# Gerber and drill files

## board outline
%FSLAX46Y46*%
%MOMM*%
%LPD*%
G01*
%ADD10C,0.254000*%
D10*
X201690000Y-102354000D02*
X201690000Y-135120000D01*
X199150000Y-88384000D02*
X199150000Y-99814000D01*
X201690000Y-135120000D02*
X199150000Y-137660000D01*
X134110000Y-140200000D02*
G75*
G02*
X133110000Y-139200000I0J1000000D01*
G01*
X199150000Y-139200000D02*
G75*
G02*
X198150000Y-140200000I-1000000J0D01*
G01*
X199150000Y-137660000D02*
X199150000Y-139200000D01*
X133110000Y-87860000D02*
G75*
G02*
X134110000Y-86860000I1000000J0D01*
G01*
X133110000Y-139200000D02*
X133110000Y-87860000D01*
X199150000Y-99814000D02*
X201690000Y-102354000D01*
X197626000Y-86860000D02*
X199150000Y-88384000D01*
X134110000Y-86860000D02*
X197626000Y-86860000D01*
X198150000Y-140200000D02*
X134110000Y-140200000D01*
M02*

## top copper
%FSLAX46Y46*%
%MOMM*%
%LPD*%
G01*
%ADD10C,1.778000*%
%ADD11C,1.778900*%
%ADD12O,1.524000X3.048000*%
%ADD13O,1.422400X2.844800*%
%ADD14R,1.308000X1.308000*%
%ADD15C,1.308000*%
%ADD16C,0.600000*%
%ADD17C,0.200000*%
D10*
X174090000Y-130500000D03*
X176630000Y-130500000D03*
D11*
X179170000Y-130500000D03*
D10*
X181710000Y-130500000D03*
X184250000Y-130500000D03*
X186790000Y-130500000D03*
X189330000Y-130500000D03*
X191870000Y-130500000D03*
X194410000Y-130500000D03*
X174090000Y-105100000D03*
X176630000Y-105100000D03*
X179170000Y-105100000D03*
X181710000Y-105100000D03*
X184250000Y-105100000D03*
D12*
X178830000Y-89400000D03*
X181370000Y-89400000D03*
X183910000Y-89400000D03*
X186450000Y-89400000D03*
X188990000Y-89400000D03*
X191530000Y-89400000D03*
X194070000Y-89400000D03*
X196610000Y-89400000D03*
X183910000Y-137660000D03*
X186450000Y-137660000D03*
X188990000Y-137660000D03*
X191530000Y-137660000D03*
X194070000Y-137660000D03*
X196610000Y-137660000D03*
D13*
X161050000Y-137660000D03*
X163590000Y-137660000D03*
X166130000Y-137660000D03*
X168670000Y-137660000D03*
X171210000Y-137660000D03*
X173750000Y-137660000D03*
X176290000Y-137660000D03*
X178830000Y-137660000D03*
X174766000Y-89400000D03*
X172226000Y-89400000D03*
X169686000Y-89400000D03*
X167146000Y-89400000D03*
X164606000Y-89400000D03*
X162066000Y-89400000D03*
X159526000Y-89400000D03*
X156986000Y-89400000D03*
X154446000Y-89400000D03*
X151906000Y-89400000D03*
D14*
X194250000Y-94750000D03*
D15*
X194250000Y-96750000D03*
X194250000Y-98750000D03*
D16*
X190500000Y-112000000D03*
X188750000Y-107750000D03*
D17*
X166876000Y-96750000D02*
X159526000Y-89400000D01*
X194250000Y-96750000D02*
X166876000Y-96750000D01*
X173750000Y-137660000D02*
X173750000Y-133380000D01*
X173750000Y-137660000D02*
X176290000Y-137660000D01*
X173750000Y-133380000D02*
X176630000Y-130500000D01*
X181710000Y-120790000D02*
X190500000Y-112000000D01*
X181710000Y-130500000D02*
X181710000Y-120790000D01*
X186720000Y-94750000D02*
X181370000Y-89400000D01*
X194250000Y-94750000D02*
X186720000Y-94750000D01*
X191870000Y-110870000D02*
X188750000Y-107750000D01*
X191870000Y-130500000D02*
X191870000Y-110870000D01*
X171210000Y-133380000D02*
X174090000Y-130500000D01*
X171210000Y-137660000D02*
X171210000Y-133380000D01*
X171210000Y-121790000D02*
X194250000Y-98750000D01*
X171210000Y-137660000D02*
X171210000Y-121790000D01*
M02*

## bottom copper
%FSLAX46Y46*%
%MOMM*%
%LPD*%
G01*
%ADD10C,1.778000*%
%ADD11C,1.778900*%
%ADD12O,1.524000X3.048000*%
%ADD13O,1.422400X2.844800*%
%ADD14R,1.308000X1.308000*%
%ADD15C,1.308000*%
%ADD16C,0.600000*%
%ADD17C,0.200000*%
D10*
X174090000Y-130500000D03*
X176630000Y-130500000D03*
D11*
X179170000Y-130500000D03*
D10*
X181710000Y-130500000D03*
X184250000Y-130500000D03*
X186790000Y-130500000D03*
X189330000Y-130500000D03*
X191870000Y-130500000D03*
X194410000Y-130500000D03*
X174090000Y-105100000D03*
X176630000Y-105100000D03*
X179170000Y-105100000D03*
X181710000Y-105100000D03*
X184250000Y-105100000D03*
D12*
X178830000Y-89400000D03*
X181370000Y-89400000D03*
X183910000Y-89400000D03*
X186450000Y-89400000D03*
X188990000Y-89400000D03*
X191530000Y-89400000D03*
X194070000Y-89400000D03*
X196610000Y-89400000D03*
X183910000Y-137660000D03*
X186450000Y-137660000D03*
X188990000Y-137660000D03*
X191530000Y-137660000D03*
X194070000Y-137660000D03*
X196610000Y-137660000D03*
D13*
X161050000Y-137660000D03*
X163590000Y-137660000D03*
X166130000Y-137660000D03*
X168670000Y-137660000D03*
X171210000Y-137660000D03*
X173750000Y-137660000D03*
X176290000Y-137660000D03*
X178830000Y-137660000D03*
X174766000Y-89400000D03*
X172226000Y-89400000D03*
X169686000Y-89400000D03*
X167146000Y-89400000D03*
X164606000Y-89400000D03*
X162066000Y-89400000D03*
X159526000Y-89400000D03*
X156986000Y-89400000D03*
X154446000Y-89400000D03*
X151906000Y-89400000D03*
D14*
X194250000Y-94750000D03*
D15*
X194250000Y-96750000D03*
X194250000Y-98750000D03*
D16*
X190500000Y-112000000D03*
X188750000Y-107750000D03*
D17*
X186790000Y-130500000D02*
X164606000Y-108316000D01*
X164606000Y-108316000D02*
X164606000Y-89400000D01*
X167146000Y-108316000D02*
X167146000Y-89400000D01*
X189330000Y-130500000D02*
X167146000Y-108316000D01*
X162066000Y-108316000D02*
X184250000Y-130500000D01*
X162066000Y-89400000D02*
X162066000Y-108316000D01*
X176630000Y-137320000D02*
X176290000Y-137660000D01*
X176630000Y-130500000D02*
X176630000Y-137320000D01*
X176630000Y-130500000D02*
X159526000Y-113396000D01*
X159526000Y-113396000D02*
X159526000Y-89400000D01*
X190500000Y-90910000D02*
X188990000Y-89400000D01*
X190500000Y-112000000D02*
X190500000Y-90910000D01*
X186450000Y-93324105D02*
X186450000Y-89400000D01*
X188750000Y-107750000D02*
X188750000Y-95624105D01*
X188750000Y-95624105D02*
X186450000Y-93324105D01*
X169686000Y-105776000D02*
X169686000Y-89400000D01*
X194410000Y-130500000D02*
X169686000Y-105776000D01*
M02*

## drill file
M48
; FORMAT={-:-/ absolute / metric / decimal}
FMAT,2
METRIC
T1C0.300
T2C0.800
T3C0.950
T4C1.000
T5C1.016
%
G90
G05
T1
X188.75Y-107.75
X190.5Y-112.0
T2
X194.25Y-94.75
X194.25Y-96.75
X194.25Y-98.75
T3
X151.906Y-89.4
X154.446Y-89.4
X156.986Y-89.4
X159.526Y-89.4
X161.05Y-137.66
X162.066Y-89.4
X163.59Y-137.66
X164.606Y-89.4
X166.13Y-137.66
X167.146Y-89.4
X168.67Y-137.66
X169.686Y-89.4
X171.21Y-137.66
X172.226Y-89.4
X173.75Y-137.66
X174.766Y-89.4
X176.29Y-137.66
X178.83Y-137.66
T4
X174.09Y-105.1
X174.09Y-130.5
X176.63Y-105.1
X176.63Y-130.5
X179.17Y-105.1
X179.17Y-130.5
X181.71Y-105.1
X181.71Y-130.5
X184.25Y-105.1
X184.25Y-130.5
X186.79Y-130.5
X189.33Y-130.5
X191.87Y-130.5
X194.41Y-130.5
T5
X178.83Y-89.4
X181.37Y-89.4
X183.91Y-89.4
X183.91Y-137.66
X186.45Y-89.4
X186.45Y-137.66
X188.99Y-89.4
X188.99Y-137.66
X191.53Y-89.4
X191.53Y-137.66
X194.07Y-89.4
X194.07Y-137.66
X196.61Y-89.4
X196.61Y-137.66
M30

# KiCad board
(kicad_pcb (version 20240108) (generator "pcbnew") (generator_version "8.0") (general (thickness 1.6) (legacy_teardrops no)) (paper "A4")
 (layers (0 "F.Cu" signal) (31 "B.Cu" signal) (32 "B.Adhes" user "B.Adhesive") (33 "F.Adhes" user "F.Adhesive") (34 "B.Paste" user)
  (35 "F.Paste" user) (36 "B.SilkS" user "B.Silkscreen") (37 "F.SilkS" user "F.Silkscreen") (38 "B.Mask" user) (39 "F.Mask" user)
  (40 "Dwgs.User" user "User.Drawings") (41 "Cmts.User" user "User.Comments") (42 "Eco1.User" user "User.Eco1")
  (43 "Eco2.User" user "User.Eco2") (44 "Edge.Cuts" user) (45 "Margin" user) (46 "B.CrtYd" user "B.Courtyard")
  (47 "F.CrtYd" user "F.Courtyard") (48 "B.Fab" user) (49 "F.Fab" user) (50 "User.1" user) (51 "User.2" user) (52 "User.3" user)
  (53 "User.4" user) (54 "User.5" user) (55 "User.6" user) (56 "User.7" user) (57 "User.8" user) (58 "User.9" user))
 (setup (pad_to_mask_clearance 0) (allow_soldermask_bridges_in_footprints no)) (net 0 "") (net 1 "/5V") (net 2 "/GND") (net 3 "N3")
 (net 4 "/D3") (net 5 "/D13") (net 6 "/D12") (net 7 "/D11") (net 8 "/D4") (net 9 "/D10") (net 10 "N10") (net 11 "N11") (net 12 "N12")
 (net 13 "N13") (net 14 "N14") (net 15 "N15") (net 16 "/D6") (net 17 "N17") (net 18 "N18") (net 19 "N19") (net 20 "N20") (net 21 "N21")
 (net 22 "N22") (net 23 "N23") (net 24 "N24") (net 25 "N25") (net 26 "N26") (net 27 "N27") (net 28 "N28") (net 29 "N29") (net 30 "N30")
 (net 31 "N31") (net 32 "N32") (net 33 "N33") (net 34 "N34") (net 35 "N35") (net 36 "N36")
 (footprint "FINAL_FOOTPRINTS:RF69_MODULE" (layer "F.Cu") (at 36.0029 13.4314)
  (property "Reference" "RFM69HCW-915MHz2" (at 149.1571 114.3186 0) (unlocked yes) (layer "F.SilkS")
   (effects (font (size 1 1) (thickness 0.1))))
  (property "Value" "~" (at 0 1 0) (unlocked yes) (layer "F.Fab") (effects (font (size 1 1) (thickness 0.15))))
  (pad "1" thru_hole circle (at 138.0871 117.0686 90) (size 1.778 1.778) (drill 1) (layers "*.Cu" "*.Mask") (remove_unused_layers no)
   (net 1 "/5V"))
  (pad "2" thru_hole circle (at 140.6271 117.0686 90) (size 1.778 1.778) (drill 1) (layers "*.Cu" "*.Mask") (remove_unused_layers no)
   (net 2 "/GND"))
  (pad "3" thru_hole circle (at 143.1671 117.0686) (size 1.7789 1.7789) (drill 1) (layers "*.Cu" "*.Mask") (remove_unused_layers no)
   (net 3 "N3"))
  (pad "4" thru_hole circle (at 145.7071 117.0686) (size 1.778 1.778) (drill 1) (layers "*.Cu" "*.Mask") (remove_unused_layers no)
   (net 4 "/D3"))
  (pad "5" thru_hole circle (at 148.2471 117.0686 90) (size 1.778 1.778) (drill 1) (layers "*.Cu" "*.Mask") (remove_unused_layers no)
   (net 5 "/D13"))
  (pad "6" thru_hole circle (at 150.7871 117.0686 90) (size 1.778 1.778) (drill 1) (layers "*.Cu" "*.Mask") (remove_unused_layers no)
   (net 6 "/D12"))
  (pad "7" thru_hole circle (at 153.3271 117.0686) (size 1.778 1.778) (drill 1) (layers "*.Cu" "*.Mask") (remove_unused_layers no)
   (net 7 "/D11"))
  (pad "8" thru_hole circle (at 155.8671 117.0686 90) (size 1.778 1.778) (drill 1) (layers "*.Cu" "*.Mask") (remove_unused_layers no)
   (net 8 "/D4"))
  (pad "9" thru_hole circle (at 158.4071 117.0686 90) (size 1.778 1.778) (drill 1) (layers "*.Cu" "*.Mask") (remove_unused_layers no)
   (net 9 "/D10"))
  (pad "10" thru_hole circle (at 138.0871 91.6686 90) (size 1.778 1.778) (drill 1) (layers "*.Cu" "*.Mask") (remove_unused_layers no)
   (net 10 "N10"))
  (pad "11" thru_hole circle (at 140.6271 91.6686 90) (size 1.778 1.778) (drill 1) (layers "*.Cu" "*.Mask") (remove_unused_layers no)
   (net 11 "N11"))
  (pad "12" thru_hole circle (at 143.1671 91.6686 90) (size 1.778 1.778) (drill 1) (layers "*.Cu" "*.Mask") (remove_unused_layers no)
   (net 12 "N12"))
  (pad "13" thru_hole circle (at 145.7071 91.6686 90) (size 1.778 1.778) (drill 1) (layers "*.Cu" "*.Mask") (remove_unused_layers no)
   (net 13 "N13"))
  (pad "14" thru_hole circle (at 148.2471 91.6686 90) (size 1.778 1.778) (drill 1) (layers "*.Cu" "*.Mask") (remove_unused_layers no)
   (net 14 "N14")))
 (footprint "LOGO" (layer "F.Cu") (at 145.75 127.75)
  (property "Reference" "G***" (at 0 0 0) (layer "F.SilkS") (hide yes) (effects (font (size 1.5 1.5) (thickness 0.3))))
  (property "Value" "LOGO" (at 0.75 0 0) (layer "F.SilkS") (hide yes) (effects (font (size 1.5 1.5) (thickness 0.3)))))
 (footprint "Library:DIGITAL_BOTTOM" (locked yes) (layer "F.Cu") (at 187.72 89.4)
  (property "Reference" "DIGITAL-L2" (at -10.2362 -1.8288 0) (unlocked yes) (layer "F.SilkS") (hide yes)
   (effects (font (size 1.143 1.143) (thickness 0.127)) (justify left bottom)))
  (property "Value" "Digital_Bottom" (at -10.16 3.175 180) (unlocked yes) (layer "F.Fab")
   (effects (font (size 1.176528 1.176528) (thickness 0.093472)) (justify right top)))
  (pad "1" thru_hole oval (at -8.89 0 90) (size 3.048 1.524) (drill 1.016) (layers "*.Cu" "*.Mask") (remove_unused_layers no) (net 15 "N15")
   (solder_mask_margin 0.0508) (thermal_bridge_angle 0))
  (pad "2" thru_hole oval (at -6.35 0 90) (size 3.048 1.524) (drill 1.016) (layers "*.Cu" "*.Mask") (remove_unused_layers no) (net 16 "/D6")
   (solder_mask_margin 0.0508) (thermal_bridge_angle 0))
  (pad "3" thru_hole oval (at -3.81 0 90) (size 3.048 1.524) (drill 1.016) (layers "*.Cu" "*.Mask") (remove_unused_layers no) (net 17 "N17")
   (solder_mask_margin 0.0508) (thermal_bridge_angle 0))
  (pad "4" thru_hole oval (at -1.27 0 90) (size 3.048 1.524) (drill 1.016) (layers "*.Cu" "*.Mask") (remove_unused_layers no) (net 8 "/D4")
   (solder_mask_margin 0.0508) (thermal_bridge_angle 0))
  (pad "5" thru_hole oval (at 1.27 0 90) (size 3.048 1.524) (drill 1.016) (layers "*.Cu" "*.Mask") (remove_unused_layers no) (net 4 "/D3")
   (solder_mask_margin 0.0508) (thermal_bridge_angle 0))
  (pad "6" thru_hole oval (at 3.81 0 90) (size 3.048 1.524) (drill 1.016) (layers "*.Cu" "*.Mask") (remove_unused_layers no) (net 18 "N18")
   (solder_mask_margin 0.0508) (thermal_bridge_angle 0))
  (pad "7" thru_hole oval (at 6.35 0 90) (size 3.048 1.524) (drill 1.016) (layers "*.Cu" "*.Mask") (remove_unused_layers no) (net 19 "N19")
   (solder_mask_margin 0.0508) (thermal_bridge_angle 0))
  (pad "8" thru_hole oval (at 8.89 0 90) (size 3.048 1.524) (drill 1.016) (layers "*.Cu" "*.Mask") (remove_unused_layers no) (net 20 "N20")
   (solder_mask_margin 0.0508) (thermal_bridge_angle 0)))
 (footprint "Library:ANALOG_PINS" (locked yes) (layer "F.Cu") (at 190.26 137.66)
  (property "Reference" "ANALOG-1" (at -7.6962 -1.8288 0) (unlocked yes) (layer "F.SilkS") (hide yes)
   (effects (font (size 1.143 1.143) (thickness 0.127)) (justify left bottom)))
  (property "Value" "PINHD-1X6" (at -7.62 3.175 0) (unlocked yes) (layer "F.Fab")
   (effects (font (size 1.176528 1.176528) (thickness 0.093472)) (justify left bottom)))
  (pad "1" thru_hole oval (at -6.35 0 90) (size 3.048 1.524) (drill 1.016) (layers "*.Cu" "*.Mask") (remove_unused_layers no) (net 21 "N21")
   (solder_mask_margin 0.0508) (thermal_bridge_angle 0))
  (pad "2" thru_hole oval (at -3.81 0 90) (size 3.048 1.524) (drill 1.016) (layers "*.Cu" "*.Mask") (remove_unused_layers no) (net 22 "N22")
   (solder_mask_margin 0.0508) (thermal_bridge_angle 0))
  (pad "3" thru_hole oval (at -1.27 0 90) (size 3.048 1.524) (drill 1.016) (layers "*.Cu" "*.Mask") (remove_unused_layers no) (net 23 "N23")
   (solder_mask_margin 0.0508) (thermal_bridge_angle 0))
  (pad "4" thru_hole oval (at 1.27 0 90) (size 3.048 1.524) (drill 1.016) (layers "*.Cu" "*.Mask") (remove_unused_layers no) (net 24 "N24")
   (solder_mask_margin 0.0508) (thermal_bridge_angle 0))
  (pad "5" thru_hole oval (at 3.81 0 90) (size 3.048 1.524) (drill 1.016) (layers "*.Cu" "*.Mask") (remove_unused_layers no) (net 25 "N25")
   (solder_mask_margin 0.0508) (thermal_bridge_angle 0))
  (pad "6" thru_hole oval (at 6.35 0 90) (size 3.048 1.524) (drill 1.016) (layers "*.Cu" "*.Mask") (remove_unused_layers no) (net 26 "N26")
   (solder_mask_margin 0.0508) (thermal_bridge_angle 0)))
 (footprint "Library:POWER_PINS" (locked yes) (layer "F.Cu") (at 169.94 137.66)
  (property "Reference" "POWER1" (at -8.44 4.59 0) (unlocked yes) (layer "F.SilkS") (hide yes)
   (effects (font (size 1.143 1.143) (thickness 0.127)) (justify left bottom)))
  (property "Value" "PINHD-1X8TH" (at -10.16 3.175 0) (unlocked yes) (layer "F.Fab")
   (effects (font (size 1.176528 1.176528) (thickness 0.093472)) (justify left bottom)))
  (pad "1" thru_hole oval (at -8.89 0 90) (size 2.8448 1.4224) (drill 0.95) (layers "*.Cu" "*.Mask") (remove_unused_layers no)
   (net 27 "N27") (solder_mask_margin 0.0508) (thermal_bridge_angle 0))
  (pad "2" thru_hole oval (at -6.35 0 90) (size 2.8448 1.4224) (drill 0.95) (layers "*.Cu" "*.Mask") (remove_unused_layers no)
   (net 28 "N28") (solder_mask_margin 0.0508) (thermal_bridge_angle 0))
  (pad "3" thru_hole oval (at -3.81 0 90) (size 2.8448 1.4224) (drill 0.95) (layers "*.Cu" "*.Mask") (remove_unused_layers no)
   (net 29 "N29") (solder_mask_margin 0.0508) (thermal_bridge_angle 0))
  (pad "4" thru_hole oval (at -1.27 0 90) (size 2.8448 1.4224) (drill 0.95) (layers "*.Cu" "*.Mask") (remove_unused_layers no)
   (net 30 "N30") (solder_mask_margin 0.0508) (thermal_bridge_angle 0))
  (pad "5" thru_hole oval (at 1.27 0 90) (size 2.8448 1.4224) (drill 0.95) (layers "*.Cu" "*.Mask") (remove_unused_layers no) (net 1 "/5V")
   (solder_mask_margin 0.0508) (thermal_bridge_angle 0))
  (pad "6" thru_hole oval (at 3.81 0 90) (size 2.8448 1.4224) (drill 0.95) (layers "*.Cu" "*.Mask") (remove_unused_layers no) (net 2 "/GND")
   (solder_mask_margin 0.0508) (thermal_bridge_angle 0))
  (pad "7" thru_hole oval (at 6.35 0 90) (size 2.8448 1.4224) (drill 0.95) (layers "*.Cu" "*.Mask") (remove_unused_layers no) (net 2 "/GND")
   (solder_mask_margin 0.0508) (thermal_bridge_angle 0))
  (pad "8" thru_hole oval (at 8.89 0 90) (size 2.8448 1.4224) (drill 0.95) (layers "*.Cu" "*.Mask") (remove_unused_layers no) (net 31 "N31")
   (solder_mask_margin 0.0508) (thermal_bridge_angle 0)))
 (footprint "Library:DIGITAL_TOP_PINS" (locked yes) (layer "F.Cu") (at 163.336 89.4 180)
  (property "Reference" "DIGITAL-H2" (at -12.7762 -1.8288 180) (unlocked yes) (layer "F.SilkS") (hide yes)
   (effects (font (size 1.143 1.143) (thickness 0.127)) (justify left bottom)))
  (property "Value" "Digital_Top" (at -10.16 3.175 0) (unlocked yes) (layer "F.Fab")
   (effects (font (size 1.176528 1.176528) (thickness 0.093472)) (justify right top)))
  (pad "1" thru_hole oval (at -11.43 0 270) (size 2.8448 1.4224) (drill 0.95) (layers "*.Cu" "*.Mask") (remove_unused_layers no)
   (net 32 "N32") (solder_mask_margin 0.0508) (thermal_bridge_angle 0))
  (pad "2" thru_hole oval (at -8.89 0 270) (size 2.8448 1.4224) (drill 0.95) (layers "*.Cu" "*.Mask") (remove_unused_layers no)
   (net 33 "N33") (solder_mask_margin 0.0508) (thermal_bridge_angle 0))
  (pad "3" thru_hole oval (at -6.35 0 270) (size 2.8448 1.4224) (drill 0.95) (layers "*.Cu" "*.Mask") (remove_unused_layers no)
   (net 9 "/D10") (solder_mask_margin 0.0508) (thermal_bridge_angle 0))
  (pad "4" thru_hole oval (at -3.81 0 270) (size 2.8448 1.4224) (drill 0.95) (layers "*.Cu" "*.Mask") (remove_unused_layers no)
   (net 7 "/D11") (solder_mask_margin 0.0508) (thermal_bridge_angle 0))
  (pad "5" thru_hole oval (at -1.27 0 270) (size 2.8448 1.4224) (drill 0.95) (layers "*.Cu" "*.Mask") (remove_unused_layers no)
   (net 6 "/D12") (solder_mask_margin 0.0508) (thermal_bridge_angle 0))
  (pad "6" thru_hole oval (at 1.27 0 270) (size 2.8448 1.4224) (drill 0.95) (layers "*.Cu" "*.Mask") (remove_unused_layers no)
   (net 5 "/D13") (solder_mask_margin 0.0508) (thermal_bridge_angle 0))
  (pad "7" thru_hole oval (at 3.81 0 270) (size 2.8448 1.4224) (drill 0.95) (layers "*.Cu" "*.Mask") (remove_unused_layers no)
   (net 2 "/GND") (solder_mask_margin 0.0508) (thermal_bridge_angle 0))
  (pad "8" thru_hole oval (at 6.35 0 270) (size 2.8448 1.4224) (drill 0.95) (layers "*.Cu" "*.Mask") (remove_unused_layers no)
   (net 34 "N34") (solder_mask_margin 0.0508) (thermal_bridge_angle 0))
  (pad "9" thru_hole oval (at 8.89 0 270) (size 2.8448 1.4224) (drill 0.95) (layers "*.Cu" "*.Mask") (remove_unused_layers no)
   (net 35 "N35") (solder_mask_margin 0.0508) (thermal_bridge_angle 0))
  (pad "10" thru_hole oval (at 11.43 0 270) (size 2.8448 1.4224) (drill 0.95) (layers "*.Cu" "*.Mask") (remove_unused_layers no)
   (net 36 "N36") (solder_mask_margin 0.0508) (thermal_bridge_angle 0)))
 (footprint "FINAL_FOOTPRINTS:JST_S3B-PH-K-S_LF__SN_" (layer "F.Cu") (at 194.25 94.75 -90)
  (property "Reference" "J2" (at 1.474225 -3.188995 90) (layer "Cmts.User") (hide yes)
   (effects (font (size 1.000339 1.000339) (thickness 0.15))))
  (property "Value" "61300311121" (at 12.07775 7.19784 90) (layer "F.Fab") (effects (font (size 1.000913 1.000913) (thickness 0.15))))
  (pad "1" thru_hole rect (at 0 0 270) (size 1.308 1.308) (drill 0.8) (layers "*.Cu" "*.Mask") (remove_unused_layers no) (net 16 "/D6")
   (solder_mask_margin 0.102))
  (pad "2" thru_hole circle (at 2 0 270) (size 1.308 1.308) (drill 0.8) (layers "*.Cu" "*.Mask") (remove_unused_layers no) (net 2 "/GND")
   (solder_mask_margin 0.102))
  (pad "3" thru_hole circle (at 4 0 270) (size 1.308 1.308) (drill 0.8) (layers "*.Cu" "*.Mask") (remove_unused_layers no) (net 1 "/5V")
   (solder_mask_margin 0.102)))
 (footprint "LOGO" (layer "B.Cu") (at 152 129.25 180)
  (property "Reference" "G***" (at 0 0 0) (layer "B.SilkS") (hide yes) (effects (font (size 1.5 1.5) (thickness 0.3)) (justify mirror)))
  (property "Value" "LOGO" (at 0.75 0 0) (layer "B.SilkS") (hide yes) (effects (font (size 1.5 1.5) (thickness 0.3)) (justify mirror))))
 (gr_line (start 201.69 102.354) (end 201.69 135.12) (stroke (width 0.254) (type solid)) (layer "Edge.Cuts"))
 (gr_line (start 199.15 88.384) (end 199.15 99.814) (stroke (width 0.254) (type solid)) (layer "Edge.Cuts"))
 (gr_line (start 201.69 135.12) (end 199.15 137.66) (stroke (width 0.254) (type solid)) (layer "Edge.Cuts"))
 (gr_arc (start 134.11 140.2) (mid 133.402893 139.907107) (end 133.11 139.2) (stroke (width 0.254) (type solid)) (layer "Edge.Cuts"))
 (gr_arc (start 199.15 139.2) (mid 198.857107 139.907107) (end 198.15 140.2) (stroke (width 0.254) (type solid)) (layer "Edge.Cuts"))
 (gr_line (start 199.15 137.66) (end 199.15 139.2) (stroke (width 0.254) (type solid)) (layer "Edge.Cuts"))
 (gr_arc (start 133.11 87.86) (mid 133.402893 87.152893) (end 134.11 86.86) (stroke (width 0.254) (type solid)) (layer "Edge.Cuts"))
 (gr_line (start 133.11 139.2) (end 133.11 87.86) (stroke (width 0.254) (type solid)) (layer "Edge.Cuts"))
 (gr_line (start 199.15 99.814) (end 201.69 102.354) (stroke (width 0.254) (type solid)) (layer "Edge.Cuts"))
 (gr_line (start 197.626 86.86) (end 199.15 88.384) (stroke (width 0.254) (type solid)) (layer "Edge.Cuts"))
 (gr_line (start 134.11 86.86) (end 197.626 86.86) (stroke (width 0.254) (type solid)) (layer "Edge.Cuts"))
 (gr_line (start 198.15 140.2) (end 134.11 140.2) (stroke (width 0.254) (type solid)) (layer "Edge.Cuts"))
 (segment (start 186.79 130.5) (end 164.606 108.316) (width 0.2) (layer "B.Cu") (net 6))
 (segment (start 164.606 108.316) (end 164.606 89.4) (width 0.2) (layer "B.Cu") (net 6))
 (segment (start 167.146 108.316) (end 167.146 89.4) (width 0.2) (layer "B.Cu") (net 7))
 (segment (start 189.33 130.5) (end 167.146 108.316) (width 0.2) (layer "B.Cu") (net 7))
 (segment (start 162.066 108.316) (end 184.25 130.5) (width 0.2) (layer "B.Cu") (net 5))
 (segment (start 162.066 89.4) (end 162.066 108.316) (width 0.2) (layer "B.Cu") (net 5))
 (segment (start 166.876 96.75) (end 159.526 89.4) (width 0.2) (layer "F.Cu") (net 2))
 (segment (start 194.25 96.75) (end 166.876 96.75) (width 0.2) (layer "F.Cu") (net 2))
 (segment (start 173.75 137.66) (end 173.75 133.38) (width 0.2) (layer "F.Cu") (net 2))
 (segment (start 173.75 137.66) (end 176.29 137.66) (width 0.2) (layer "F.Cu") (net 2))
 (segment (start 173.75 133.38) (end 176.63 130.5) (width 0.2) (layer "F.Cu") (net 2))
 (segment (start 176.63 137.32) (end 176.29 137.66) (width 0.2) (layer "B.Cu") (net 2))
 (segment (start 176.63 130.5) (end 176.63 137.32) (width 0.2) (layer "B.Cu") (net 2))
 (segment (start 176.63 130.5) (end 159.526 113.396) (width 0.2) (layer "B.Cu") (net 2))
 (segment (start 159.526 113.396) (end 159.526 89.4) (width 0.2) (layer "B.Cu") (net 2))
 (segment (start 181.71 120.79) (end 190.5 112) (width 0.2) (layer "F.Cu") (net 4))
 (segment (start 181.71 130.5) (end 181.71 120.79) (width 0.2) (layer "F.Cu") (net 4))
 (via (at 190.5 112) (size 0.6) (drill 0.3) (layers "F.Cu" "B.Cu") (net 4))
 (segment (start 190.5 90.91) (end 188.99 89.4) (width 0.2) (layer "B.Cu") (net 4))
 (segment (start 190.5 112) (end 190.5 90.91) (width 0.2) (layer "B.Cu") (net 4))
 (segment (start 186.72 94.75) (end 181.37 89.4) (width 0.2) (layer "F.Cu") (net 16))
 (segment (start 194.25 94.75) (end 186.72 94.75) (width 0.2) (layer "F.Cu") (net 16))
 (segment (start 191.87 110.87) (end 188.75 107.75) (width 0.2) (layer "F.Cu") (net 8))
 (segment (start 191.87 130.5) (end 191.87 110.87) (width 0.2) (layer "F.Cu") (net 8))
 (via (at 188.75 107.75) (size 0.6) (drill 0.3) (layers "F.Cu" "B.Cu") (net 8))
 (segment (start 186.45 93.324105) (end 186.45 89.4) (width 0.2) (layer "B.Cu") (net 8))
 (segment (start 188.75 107.75) (end 188.75 95.624105) (width 0.2) (layer "B.Cu") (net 8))
 (segment (start 188.75 95.624105) (end 186.45 93.324105) (width 0.2) (layer "B.Cu") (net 8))
 (segment (start 171.21 133.38) (end 174.09 130.5) (width 0.2) (layer "F.Cu") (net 1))
 (segment (start 171.21 137.66) (end 171.21 133.38) (width 0.2) (layer "F.Cu") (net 1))
 (segment (start 171.21 121.79) (end 194.25 98.75) (width 0.2) (layer "F.Cu") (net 1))
 (segment (start 171.21 137.66) (end 171.21 121.79) (width 0.2) (layer "F.Cu") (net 1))
 (segment (start 169.686 105.776) (end 169.686 89.4) (width 0.2) (layer "B.Cu") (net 9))
 (segment (start 194.41 130.5) (end 169.686 105.776) (width 0.2) (layer "B.Cu") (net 9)))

